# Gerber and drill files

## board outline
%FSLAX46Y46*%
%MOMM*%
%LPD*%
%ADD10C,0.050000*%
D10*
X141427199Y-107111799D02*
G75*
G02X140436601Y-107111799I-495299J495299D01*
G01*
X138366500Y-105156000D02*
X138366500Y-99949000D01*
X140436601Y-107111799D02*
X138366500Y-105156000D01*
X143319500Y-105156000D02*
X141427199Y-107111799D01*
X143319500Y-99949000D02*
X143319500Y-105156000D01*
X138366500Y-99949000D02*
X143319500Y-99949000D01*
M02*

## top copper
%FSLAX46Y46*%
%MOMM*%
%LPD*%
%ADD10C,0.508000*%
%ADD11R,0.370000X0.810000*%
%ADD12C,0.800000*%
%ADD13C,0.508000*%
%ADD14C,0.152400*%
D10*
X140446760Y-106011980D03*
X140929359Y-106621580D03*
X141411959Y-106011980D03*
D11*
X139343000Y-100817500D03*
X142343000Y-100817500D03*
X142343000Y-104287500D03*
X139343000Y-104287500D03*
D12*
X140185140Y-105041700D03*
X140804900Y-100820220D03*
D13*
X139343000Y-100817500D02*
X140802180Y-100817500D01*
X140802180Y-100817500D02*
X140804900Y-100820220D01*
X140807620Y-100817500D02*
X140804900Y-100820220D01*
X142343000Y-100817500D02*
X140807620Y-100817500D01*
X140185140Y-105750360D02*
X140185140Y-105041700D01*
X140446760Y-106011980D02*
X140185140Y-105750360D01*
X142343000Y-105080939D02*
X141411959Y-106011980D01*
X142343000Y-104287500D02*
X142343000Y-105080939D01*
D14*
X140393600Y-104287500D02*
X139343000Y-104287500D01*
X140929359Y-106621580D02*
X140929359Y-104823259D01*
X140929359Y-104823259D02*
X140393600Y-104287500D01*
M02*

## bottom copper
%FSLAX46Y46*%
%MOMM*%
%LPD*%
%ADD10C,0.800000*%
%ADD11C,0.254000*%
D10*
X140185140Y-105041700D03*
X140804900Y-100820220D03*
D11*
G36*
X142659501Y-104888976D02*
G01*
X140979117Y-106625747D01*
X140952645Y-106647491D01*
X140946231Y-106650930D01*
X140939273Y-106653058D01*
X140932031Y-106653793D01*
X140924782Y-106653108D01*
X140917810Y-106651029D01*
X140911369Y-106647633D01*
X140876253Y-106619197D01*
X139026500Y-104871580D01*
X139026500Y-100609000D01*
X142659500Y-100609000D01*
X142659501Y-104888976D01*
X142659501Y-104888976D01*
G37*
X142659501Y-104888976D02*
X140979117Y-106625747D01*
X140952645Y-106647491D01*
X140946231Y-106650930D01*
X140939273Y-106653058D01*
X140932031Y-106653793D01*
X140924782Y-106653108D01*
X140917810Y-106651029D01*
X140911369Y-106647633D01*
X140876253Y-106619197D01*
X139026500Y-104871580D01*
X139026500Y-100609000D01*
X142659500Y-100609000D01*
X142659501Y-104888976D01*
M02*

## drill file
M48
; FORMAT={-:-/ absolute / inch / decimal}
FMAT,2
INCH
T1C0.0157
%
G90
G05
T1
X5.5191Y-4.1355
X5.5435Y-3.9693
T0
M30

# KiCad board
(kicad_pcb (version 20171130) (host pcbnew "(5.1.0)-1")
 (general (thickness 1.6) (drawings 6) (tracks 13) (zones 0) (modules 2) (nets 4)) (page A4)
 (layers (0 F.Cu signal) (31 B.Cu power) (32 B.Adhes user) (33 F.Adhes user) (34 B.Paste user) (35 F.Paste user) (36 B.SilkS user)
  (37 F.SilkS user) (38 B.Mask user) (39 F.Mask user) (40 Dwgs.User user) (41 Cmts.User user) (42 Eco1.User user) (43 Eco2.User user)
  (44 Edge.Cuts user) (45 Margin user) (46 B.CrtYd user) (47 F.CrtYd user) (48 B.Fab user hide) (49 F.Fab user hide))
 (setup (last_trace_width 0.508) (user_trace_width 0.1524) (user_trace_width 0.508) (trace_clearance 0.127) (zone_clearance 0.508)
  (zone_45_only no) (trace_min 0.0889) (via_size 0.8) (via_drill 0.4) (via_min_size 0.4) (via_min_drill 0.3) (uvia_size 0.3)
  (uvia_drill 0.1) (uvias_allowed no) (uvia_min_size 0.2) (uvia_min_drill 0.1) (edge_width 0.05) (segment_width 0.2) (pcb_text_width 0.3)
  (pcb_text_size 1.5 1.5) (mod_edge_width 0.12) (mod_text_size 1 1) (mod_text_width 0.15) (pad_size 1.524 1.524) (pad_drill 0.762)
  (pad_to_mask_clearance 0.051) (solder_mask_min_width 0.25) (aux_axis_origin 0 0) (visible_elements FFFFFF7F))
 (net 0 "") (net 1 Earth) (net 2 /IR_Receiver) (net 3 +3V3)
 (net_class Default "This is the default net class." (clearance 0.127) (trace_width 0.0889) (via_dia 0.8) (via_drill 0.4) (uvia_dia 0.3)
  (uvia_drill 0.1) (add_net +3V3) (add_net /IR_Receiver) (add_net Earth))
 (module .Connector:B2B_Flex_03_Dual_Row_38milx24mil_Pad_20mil (layer F.Cu) (at 140.44676 106.01198)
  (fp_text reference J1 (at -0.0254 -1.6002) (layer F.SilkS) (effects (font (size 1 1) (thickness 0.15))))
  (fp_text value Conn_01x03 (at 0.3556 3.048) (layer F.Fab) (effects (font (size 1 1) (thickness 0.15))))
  (pad 1 smd circle (at 0 0) (size 0.508 0.508) (layers F.Cu F.Paste F.Mask) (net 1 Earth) (zone_connect 0))
  (pad 2 smd circle (at 0.482599 0.6096) (size 0.508 0.508) (layers F.Cu F.Paste F.Mask) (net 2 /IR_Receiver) (zone_connect 0))
  (pad 3 smd circle (at 0.965199 0) (size 0.508 0.508) (layers F.Cu F.Paste F.Mask) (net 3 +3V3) (zone_connect 0)))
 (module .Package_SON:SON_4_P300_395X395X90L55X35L (layer F.Cu) (at 140.843 102.5525)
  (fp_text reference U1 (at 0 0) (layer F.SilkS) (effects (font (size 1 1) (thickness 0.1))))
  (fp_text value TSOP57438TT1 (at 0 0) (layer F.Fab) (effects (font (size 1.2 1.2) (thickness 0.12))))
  (pad 8 smd rect (at -1.5 -1.735 90) (size 0.81 0.37) (layers F.Cu F.Paste F.Mask) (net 1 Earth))
  (pad 6 smd rect (at 1.5 -1.735 90) (size 0.81 0.37) (layers F.Cu F.Paste F.Mask) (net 1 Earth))
  (pad 5 smd rect (at 1.5 1.735 90) (size 0.81 0.37) (layers F.Cu F.Paste F.Mask) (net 3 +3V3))
  (pad 1 smd rect (at -1.5 1.735 90) (size 0.81 0.37) (layers F.Cu F.Paste F.Mask) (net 2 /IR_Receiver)))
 (gr_arc (start 140.9319 106.6165) (end 140.436601 107.111799) (angle -90) (layer Edge.Cuts) (width 0.05))
 (gr_line (start 138.3665 105.156) (end 138.3665 99.949) (layer Edge.Cuts) (width 0.05))
 (gr_line (start 140.436601 107.111799) (end 138.3665 105.156) (layer Edge.Cuts) (width 0.05))
 (gr_line (start 143.3195 105.156) (end 141.427199 107.111799) (layer Edge.Cuts) (width 0.05))
 (gr_line (start 143.3195 99.949) (end 143.3195 105.156) (layer Edge.Cuts) (width 0.05))
 (gr_line (start 138.3665 99.949) (end 143.3195 99.949) (layer Edge.Cuts) (width 0.05))
 (via (at 140.18514 105.0417) (size 0.8) (drill 0.4) (layers F.Cu B.Cu) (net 1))
 (via (at 140.8049 100.82022) (size 0.8) (drill 0.4) (layers F.Cu B.Cu) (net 1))
 (segment (start 139.343 100.8175) (end 140.80218 100.8175) (width 0.508) (layer F.Cu) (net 1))
 (segment (start 140.80218 100.8175) (end 140.8049 100.82022) (width 0.508) (layer F.Cu) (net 1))
 (segment (start 140.80762 100.8175) (end 140.8049 100.82022) (width 0.508) (layer F.Cu) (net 1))
 (segment (start 142.343 100.8175) (end 140.80762 100.8175) (width 0.508) (layer F.Cu) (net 1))
 (segment (start 140.18514 105.75036) (end 140.18514 105.0417) (width 0.508) (layer F.Cu) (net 1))
 (segment (start 140.44676 106.01198) (end 140.18514 105.75036) (width 0.508) (layer F.Cu) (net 1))
 (segment (start 142.343 105.080939) (end 141.411959 106.01198) (width 0.508) (layer F.Cu) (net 3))
 (segment (start 142.343 104.2875) (end 142.343 105.080939) (width 0.508) (layer F.Cu) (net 3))
 (segment (start 140.3936 104.2875) (end 139.343 104.2875) (width 0.1524) (layer F.Cu) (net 2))
 (segment (start 140.929359 106.62158) (end 140.929359 104.823259) (width 0.1524) (layer F.Cu) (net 2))
 (segment (start 140.929359 104.823259) (end 140.3936 104.2875) (width 0.1524) (layer F.Cu) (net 2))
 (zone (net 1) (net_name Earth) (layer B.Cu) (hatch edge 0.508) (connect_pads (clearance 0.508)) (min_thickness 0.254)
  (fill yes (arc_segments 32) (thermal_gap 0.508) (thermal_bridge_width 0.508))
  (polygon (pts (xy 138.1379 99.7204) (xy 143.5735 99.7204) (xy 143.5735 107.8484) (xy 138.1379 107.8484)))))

